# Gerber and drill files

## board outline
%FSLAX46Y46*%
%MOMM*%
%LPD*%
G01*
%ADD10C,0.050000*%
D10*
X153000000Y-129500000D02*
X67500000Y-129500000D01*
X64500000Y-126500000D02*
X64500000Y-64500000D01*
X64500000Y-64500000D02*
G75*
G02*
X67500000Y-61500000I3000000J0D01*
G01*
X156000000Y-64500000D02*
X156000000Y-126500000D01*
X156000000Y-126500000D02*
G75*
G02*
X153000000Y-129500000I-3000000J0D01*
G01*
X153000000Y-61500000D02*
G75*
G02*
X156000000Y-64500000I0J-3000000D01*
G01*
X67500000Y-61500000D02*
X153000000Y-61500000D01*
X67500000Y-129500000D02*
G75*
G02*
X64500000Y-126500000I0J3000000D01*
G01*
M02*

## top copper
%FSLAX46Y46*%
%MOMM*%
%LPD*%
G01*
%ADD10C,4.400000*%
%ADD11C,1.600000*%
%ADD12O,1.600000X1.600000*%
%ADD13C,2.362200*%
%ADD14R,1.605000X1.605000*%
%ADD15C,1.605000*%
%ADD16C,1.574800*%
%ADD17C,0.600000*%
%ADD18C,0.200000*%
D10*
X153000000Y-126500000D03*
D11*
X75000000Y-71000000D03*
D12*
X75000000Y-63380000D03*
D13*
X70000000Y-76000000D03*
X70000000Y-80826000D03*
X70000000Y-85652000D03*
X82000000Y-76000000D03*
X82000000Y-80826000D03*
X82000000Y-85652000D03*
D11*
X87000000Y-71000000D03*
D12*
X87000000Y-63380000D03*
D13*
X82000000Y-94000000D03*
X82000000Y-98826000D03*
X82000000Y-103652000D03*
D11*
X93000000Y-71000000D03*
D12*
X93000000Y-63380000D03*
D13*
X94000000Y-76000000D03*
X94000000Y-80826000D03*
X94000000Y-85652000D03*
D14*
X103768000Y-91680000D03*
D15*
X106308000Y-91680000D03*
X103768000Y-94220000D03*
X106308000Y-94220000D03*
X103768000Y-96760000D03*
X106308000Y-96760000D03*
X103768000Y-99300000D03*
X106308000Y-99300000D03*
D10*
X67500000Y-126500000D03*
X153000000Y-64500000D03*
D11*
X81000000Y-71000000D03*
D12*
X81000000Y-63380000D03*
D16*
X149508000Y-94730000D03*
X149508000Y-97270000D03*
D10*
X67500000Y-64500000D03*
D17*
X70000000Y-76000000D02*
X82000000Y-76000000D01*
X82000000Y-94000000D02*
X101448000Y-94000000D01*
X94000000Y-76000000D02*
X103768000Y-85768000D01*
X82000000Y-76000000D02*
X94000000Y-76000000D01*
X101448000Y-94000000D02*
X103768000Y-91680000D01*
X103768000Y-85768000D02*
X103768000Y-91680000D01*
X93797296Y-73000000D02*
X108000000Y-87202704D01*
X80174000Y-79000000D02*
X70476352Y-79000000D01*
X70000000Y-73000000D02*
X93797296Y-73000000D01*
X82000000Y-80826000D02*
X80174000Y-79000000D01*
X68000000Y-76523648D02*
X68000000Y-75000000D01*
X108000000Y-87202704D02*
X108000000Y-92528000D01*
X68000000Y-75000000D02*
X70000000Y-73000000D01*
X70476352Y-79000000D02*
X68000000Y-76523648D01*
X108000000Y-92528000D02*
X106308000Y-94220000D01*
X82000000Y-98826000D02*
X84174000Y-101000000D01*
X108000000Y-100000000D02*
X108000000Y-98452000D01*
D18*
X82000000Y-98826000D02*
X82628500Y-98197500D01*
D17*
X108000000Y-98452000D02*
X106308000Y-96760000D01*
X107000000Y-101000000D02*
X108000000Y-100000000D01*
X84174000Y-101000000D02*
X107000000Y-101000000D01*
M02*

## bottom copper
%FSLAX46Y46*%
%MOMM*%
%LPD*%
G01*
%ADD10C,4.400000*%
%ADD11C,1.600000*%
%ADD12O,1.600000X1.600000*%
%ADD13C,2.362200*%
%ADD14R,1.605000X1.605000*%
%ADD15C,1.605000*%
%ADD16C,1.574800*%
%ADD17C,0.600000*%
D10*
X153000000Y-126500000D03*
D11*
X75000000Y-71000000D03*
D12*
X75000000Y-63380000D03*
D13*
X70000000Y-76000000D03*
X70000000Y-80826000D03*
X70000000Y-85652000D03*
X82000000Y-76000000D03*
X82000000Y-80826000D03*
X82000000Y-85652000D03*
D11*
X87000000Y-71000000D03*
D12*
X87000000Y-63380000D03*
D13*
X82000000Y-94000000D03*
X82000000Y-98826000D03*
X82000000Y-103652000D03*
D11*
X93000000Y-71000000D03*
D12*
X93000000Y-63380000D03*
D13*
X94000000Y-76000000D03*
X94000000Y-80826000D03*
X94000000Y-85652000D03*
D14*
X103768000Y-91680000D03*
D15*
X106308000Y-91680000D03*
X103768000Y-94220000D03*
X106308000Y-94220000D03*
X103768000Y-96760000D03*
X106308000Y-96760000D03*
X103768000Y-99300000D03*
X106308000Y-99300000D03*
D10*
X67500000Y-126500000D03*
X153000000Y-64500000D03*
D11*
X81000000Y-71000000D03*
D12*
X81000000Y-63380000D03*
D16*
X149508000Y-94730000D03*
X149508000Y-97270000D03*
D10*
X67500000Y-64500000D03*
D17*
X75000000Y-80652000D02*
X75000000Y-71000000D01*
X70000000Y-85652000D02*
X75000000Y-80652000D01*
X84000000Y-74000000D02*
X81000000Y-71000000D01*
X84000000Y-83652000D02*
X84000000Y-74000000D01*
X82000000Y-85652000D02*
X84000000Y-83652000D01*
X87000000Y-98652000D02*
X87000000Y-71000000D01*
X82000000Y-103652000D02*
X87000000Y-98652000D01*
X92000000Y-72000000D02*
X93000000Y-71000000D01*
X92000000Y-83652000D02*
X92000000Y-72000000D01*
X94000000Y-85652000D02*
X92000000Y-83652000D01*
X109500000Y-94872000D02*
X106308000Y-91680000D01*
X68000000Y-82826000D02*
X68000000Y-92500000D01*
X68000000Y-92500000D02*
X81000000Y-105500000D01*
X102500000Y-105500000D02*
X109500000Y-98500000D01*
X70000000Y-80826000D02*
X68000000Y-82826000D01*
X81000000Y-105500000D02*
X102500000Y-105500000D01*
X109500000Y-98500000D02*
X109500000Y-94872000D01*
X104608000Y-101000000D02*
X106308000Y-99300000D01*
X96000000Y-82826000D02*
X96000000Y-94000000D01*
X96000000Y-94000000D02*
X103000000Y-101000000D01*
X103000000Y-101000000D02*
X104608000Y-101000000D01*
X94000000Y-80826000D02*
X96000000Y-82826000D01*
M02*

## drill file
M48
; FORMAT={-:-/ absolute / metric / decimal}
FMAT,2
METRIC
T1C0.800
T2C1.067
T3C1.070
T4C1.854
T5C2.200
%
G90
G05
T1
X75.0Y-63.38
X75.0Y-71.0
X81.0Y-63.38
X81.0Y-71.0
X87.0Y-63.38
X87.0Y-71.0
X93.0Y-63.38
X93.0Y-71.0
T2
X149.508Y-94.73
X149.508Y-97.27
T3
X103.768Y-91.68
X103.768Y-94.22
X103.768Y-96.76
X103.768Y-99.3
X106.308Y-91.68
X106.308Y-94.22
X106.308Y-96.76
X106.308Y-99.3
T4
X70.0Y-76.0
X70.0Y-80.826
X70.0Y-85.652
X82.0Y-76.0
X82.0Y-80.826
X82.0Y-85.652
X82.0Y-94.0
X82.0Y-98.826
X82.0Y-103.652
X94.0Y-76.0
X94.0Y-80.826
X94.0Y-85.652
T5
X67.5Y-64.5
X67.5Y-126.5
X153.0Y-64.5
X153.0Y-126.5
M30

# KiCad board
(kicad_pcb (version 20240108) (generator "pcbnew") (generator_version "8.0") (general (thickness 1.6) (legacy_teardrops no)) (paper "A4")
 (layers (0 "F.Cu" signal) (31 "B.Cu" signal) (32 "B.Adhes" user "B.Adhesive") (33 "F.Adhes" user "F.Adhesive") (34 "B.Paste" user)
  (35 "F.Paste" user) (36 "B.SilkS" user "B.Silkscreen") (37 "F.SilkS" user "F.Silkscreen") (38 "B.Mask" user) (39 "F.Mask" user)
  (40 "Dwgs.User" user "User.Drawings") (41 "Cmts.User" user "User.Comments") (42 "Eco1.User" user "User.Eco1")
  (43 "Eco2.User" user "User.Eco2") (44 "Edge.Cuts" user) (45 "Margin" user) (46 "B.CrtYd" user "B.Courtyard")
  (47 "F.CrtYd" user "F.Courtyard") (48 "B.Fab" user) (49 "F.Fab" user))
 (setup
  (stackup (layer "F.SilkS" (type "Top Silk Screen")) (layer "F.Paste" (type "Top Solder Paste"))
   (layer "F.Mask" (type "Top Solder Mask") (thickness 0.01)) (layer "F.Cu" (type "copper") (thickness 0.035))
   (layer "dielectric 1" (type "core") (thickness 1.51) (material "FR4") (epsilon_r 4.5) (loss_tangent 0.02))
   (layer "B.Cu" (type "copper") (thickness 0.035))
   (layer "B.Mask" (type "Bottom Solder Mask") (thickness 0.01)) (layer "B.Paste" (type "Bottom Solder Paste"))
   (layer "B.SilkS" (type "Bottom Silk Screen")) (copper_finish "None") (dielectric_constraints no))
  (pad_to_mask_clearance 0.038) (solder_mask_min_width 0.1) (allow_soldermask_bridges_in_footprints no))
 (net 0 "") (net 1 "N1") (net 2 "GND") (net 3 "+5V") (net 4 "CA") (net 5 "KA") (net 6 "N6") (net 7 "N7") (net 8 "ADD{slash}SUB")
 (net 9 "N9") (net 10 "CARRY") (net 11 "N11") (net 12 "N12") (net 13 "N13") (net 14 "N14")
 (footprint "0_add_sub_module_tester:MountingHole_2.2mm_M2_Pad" (layer "F.Cu") (at 153 126.5)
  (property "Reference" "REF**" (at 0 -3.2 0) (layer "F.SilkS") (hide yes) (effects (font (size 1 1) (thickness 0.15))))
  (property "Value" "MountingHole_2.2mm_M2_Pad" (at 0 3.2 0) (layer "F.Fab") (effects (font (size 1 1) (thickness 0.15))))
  (pad "1" thru_hole circle (at 0 0) (size 4.4 4.4) (drill 2.2) (layers "*.Cu" "*.Mask") (remove_unused_layers no)))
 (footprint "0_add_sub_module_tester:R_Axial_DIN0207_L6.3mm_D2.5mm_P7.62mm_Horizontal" (layer "F.Cu") (at 75 71 90)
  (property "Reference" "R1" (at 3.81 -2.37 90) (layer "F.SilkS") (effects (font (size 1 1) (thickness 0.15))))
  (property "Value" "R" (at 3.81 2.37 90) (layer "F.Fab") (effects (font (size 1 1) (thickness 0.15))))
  (pad "1" thru_hole circle (at 0 0 90) (size 1.6 1.6) (drill 0.8) (layers "*.Cu" "*.Mask") (remove_unused_layers no) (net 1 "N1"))
  (pad "2" thru_hole oval (at 7.62 0 90) (size 1.6 1.6) (drill 0.8) (layers "*.Cu" "*.Mask") (remove_unused_layers no) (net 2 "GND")))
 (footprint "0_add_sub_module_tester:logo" (layer "F.Cu") (at 127 95.5)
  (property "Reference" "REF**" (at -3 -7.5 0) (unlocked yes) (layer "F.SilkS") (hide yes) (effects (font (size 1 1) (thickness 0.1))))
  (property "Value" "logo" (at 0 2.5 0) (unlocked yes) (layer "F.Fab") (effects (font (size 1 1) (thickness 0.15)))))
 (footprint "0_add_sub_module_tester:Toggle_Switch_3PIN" (layer "F.Cu") (at 70 76 -90)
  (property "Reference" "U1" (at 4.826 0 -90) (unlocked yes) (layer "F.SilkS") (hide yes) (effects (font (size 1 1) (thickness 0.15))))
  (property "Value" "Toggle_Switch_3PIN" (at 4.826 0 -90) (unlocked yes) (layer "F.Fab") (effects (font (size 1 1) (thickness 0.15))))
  (pad "1" thru_hole circle (at 0 0 270) (size 2.3622 2.3622) (drill 1.8542) (layers "*.Cu" "*.Mask") (remove_unused_layers no)
   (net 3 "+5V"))
  (pad "2" thru_hole circle (at 4.826 0 270) (size 2.3622 2.3622) (drill 1.8542) (layers "*.Cu" "*.Mask") (remove_unused_layers no)
   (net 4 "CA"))
  (pad "3" thru_hole circle (at 9.652 0 270) (size 2.3622 2.3622) (drill 1.8542) (layers "*.Cu" "*.Mask") (remove_unused_layers no)
   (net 1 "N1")))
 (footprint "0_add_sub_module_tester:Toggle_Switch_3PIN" (layer "F.Cu") (at 82 76 -90)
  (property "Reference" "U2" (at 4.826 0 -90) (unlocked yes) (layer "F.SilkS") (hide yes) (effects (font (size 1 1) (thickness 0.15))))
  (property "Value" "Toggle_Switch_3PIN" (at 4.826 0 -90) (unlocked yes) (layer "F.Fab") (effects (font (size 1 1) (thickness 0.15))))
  (pad "1" thru_hole circle (at 0 0 270) (size 2.3622 2.3622) (drill 1.8542) (layers "*.Cu" "*.Mask") (remove_unused_layers no)
   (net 3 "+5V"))
  (pad "2" thru_hole circle (at 4.826 0 270) (size 2.3622 2.3622) (drill 1.8542) (layers "*.Cu" "*.Mask") (remove_unused_layers no)
   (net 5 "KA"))
  (pad "3" thru_hole circle (at 9.652 0 270) (size 2.3622 2.3622) (drill 1.8542) (layers "*.Cu" "*.Mask") (remove_unused_layers no)
   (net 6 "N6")))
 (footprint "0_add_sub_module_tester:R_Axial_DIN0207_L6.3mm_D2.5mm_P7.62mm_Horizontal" (layer "F.Cu") (at 87 71 90)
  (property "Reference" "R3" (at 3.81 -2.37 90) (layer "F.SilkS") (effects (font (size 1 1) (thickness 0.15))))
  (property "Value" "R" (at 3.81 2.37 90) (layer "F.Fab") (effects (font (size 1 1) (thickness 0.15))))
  (pad "1" thru_hole circle (at 0 0 90) (size 1.6 1.6) (drill 0.8) (layers "*.Cu" "*.Mask") (remove_unused_layers no) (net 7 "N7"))
  (pad "2" thru_hole oval (at 7.62 0 90) (size 1.6 1.6) (drill 0.8) (layers "*.Cu" "*.Mask") (remove_unused_layers no) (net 2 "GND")))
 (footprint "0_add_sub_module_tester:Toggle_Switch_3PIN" (layer "F.Cu") (at 82 94 -90)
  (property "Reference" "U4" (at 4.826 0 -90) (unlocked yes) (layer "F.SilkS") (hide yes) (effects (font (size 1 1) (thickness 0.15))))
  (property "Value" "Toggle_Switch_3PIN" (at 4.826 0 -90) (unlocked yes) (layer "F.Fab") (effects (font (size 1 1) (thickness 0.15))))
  (pad "1" thru_hole circle (at 0 0 270) (size 2.3622 2.3622) (drill 1.8542) (layers "*.Cu" "*.Mask") (remove_unused_layers no)
   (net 3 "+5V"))
  (pad "2" thru_hole circle (at 4.826 0 270) (size 2.3622 2.3622) (drill 1.8542) (layers "*.Cu" "*.Mask") (remove_unused_layers no)
   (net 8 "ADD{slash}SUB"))
  (pad "3" thru_hole circle (at 9.652 0 270) (size 2.3622 2.3622) (drill 1.8542) (layers "*.Cu" "*.Mask") (remove_unused_layers no)
   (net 7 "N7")))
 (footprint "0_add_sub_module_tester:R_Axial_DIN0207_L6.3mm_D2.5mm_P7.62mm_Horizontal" (layer "F.Cu") (at 93 71 90)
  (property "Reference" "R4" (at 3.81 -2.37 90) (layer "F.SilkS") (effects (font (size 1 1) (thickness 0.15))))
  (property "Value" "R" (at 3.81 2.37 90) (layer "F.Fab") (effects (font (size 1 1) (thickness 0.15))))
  (pad "1" thru_hole circle (at 0 0 90) (size 1.6 1.6) (drill 0.8) (layers "*.Cu" "*.Mask") (remove_unused_layers no) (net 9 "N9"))
  (pad "2" thru_hole oval (at 7.62 0 90) (size 1.6 1.6) (drill 0.8) (layers "*.Cu" "*.Mask") (remove_unused_layers no) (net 2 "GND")))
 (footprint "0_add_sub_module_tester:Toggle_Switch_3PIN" (layer "F.Cu") (at 94 76 -90)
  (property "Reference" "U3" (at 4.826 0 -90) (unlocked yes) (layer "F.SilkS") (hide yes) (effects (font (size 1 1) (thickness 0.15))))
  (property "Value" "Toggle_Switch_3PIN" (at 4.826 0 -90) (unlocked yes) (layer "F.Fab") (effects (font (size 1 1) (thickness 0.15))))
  (pad "1" thru_hole circle (at 0 0 270) (size 2.3622 2.3622) (drill 1.8542) (layers "*.Cu" "*.Mask") (remove_unused_layers no)
   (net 3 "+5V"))
  (pad "2" thru_hole circle (at 4.826 0 270) (size 2.3622 2.3622) (drill 1.8542) (layers "*.Cu" "*.Mask") (remove_unused_layers no)
   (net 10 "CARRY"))
  (pad "3" thru_hole circle (at 9.652 0 270) (size 2.3622 2.3622) (drill 1.8542) (layers "*.Cu" "*.Mask") (remove_unused_layers no)
   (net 9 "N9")))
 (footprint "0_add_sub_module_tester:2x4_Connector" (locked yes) (layer "F.Cu") (at 103.738 91.69 -90)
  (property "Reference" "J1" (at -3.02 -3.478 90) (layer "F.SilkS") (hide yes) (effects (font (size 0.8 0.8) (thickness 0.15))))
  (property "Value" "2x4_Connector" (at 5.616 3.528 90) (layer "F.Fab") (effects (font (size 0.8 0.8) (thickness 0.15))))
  (pad "1" thru_hole rect (at -0.01 -0.03 270) (size 1.605 1.605) (drill 1.07) (layers "*.Cu" "*.Mask") (remove_unused_layers no)
   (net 3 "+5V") (solder_mask_margin 0.102))
  (pad "2" thru_hole circle (at -0.01 -2.57 270) (size 1.605 1.605) (drill 1.07) (layers "*.Cu" "*.Mask") (remove_unused_layers no)
   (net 4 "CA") (solder_mask_margin 0.102))
  (pad "3" thru_hole circle (at 2.53 -0.03 270) (size 1.605 1.605) (drill 1.07) (layers "*.Cu" "*.Mask") (remove_unused_layers no)
   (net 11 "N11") (solder_mask_margin 0.102))
  (pad "4" thru_hole circle (at 2.53 -2.57 270) (size 1.605 1.605) (drill 1.07) (layers "*.Cu" "*.Mask") (remove_unused_layers no)
   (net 5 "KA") (solder_mask_margin 0.102))
  (pad "5" thru_hole circle (at 5.07 -0.03 270) (size 1.605 1.605) (drill 1.07) (layers "*.Cu" "*.Mask") (remove_unused_layers no)
   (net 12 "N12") (solder_mask_margin 0.102))
  (pad "6" thru_hole circle (at 5.07 -2.57 270) (size 1.605 1.605) (drill 1.07) (layers "*.Cu" "*.Mask") (remove_unused_layers no)
   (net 8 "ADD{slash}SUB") (solder_mask_margin 0.102))
  (pad "7" thru_hole circle (at 7.61 -0.03 270) (size 1.605 1.605) (drill 1.07) (layers "*.Cu" "*.Mask") (remove_unused_layers no)
   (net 2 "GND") (solder_mask_margin 0.102))
  (pad "8" thru_hole circle (at 7.61 -2.57 270) (size 1.605 1.605) (drill 1.07) (layers "*.Cu" "*.Mask") (remove_unused_layers no)
   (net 10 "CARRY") (solder_mask_margin 0.102)))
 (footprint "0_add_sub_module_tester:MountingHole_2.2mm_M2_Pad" (layer "F.Cu") (at 67.5 126.5)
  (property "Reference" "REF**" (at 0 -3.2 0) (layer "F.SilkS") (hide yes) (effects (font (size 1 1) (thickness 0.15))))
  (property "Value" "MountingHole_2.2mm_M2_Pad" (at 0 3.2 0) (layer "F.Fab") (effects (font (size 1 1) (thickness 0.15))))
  (pad "1" thru_hole circle (at 0 0) (size 4.4 4.4) (drill 2.2) (layers "*.Cu" "*.Mask") (remove_unused_layers no)))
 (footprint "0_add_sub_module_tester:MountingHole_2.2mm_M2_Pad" (layer "F.Cu") (at 153 64.5)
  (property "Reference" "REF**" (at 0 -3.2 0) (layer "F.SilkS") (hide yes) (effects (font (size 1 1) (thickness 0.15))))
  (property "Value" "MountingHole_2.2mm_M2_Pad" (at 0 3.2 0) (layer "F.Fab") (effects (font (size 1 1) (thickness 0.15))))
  (pad "1" thru_hole circle (at 0 0) (size 4.4 4.4) (drill 2.2) (layers "*.Cu" "*.Mask") (remove_unused_layers no)))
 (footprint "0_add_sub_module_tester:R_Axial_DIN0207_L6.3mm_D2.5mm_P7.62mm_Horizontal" (layer "F.Cu") (at 81 71 90)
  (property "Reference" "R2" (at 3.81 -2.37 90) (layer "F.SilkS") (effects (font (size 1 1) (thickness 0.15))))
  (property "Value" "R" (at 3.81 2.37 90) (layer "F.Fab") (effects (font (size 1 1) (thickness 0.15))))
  (pad "1" thru_hole circle (at 0 0 90) (size 1.6 1.6) (drill 0.8) (layers "*.Cu" "*.Mask") (remove_unused_layers no) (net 6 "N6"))
  (pad "2" thru_hole oval (at 7.62 0 90) (size 1.6 1.6) (drill 0.8) (layers "*.Cu" "*.Mask") (remove_unused_layers no) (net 2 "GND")))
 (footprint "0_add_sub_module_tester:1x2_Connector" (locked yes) (layer "F.Cu") (at 149.508 94.73 -90)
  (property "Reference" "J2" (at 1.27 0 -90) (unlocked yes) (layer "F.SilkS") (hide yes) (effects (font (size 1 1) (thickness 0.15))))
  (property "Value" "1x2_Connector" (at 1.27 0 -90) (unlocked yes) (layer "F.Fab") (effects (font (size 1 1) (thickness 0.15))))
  (pad "1" thru_hole circle (at 0 0 270) (size 1.5748 1.5748) (drill 1.0668) (layers "*.Cu" "*.Mask") (remove_unused_layers no)
   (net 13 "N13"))
  (pad "2" thru_hole circle (at 2.54 0 270) (size 1.5748 1.5748) (drill 1.0668) (layers "*.Cu" "*.Mask") (remove_unused_layers no)
   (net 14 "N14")))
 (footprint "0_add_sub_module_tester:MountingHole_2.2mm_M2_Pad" (layer "F.Cu") (at 67.5 64.5)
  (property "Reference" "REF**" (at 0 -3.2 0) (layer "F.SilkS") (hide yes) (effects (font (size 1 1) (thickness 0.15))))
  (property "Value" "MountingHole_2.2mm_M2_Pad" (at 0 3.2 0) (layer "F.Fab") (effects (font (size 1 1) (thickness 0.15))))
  (pad "1" thru_hole circle (at 0 0) (size 4.4 4.4) (drill 2.2) (layers "*.Cu" "*.Mask") (remove_unused_layers no)))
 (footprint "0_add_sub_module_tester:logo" (layer "B.Cu") (at 129.5 95.5 180)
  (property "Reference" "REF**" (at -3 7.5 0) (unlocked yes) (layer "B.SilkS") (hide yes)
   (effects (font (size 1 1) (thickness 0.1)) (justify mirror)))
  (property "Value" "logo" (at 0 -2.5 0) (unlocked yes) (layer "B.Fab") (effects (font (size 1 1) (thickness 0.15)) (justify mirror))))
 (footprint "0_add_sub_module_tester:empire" (layer "B.Cu") (at 141 112 180)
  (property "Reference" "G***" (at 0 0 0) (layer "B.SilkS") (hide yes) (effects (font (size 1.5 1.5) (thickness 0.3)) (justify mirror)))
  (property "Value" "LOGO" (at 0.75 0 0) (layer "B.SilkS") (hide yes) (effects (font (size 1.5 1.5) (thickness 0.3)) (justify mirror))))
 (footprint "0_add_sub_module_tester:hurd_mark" (layer "B.Cu") (at 106 68.75 180)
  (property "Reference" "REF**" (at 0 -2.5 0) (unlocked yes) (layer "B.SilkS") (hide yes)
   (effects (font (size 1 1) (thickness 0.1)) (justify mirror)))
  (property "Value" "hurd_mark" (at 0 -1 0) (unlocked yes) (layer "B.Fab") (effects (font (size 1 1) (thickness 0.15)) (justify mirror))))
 (gr_line (start 153 129.5) (end 67.5 129.5) (stroke (width 0.05) (type default)) (layer "Edge.Cuts"))
 (gr_line (start 64.5 126.5) (end 64.5 64.5) (stroke (width 0.05) (type default)) (layer "Edge.Cuts"))
 (gr_arc (start 64.5 64.5) (mid 65.37868 62.37868) (end 67.5 61.5) (stroke (width 0.05) (type default)) (layer "Edge.Cuts"))
 (gr_line (start 156 64.5) (end 156 126.5) (stroke (width 0.05) (type default)) (layer "Edge.Cuts"))
 (gr_arc (start 156 126.5) (mid 155.12132 128.62132) (end 153 129.5) (stroke (width 0.05) (type default)) (layer "Edge.Cuts"))
 (gr_arc (start 153 61.5) (mid 155.12132 62.37868) (end 156 64.5) (stroke (width 0.05) (type default)) (layer "Edge.Cuts"))
 (gr_line (start 67.5 61.5) (end 153 61.5) (stroke (width 0.05) (type default)) (layer "Edge.Cuts"))
 (gr_arc (start 67.5 129.5) (mid 65.37868 128.62132) (end 64.5 126.5) (stroke (width 0.05) (type default)) (layer "Edge.Cuts"))
 (segment (start 75 80.652) (end 75 71) (width 0.6) (layer "B.Cu") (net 1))
 (segment (start 70 85.652) (end 75 80.652) (width 0.6) (layer "B.Cu") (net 1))
 (segment (start 84 74) (end 81 71) (width 0.6) (layer "B.Cu") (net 6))
 (segment (start 84 83.652) (end 84 74) (width 0.6) (layer "B.Cu") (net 6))
 (segment (start 82 85.652) (end 84 83.652) (width 0.6) (layer "B.Cu") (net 6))
 (segment (start 87 98.652) (end 87 71) (width 0.6) (layer "B.Cu") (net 7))
 (segment (start 82 103.652) (end 87 98.652) (width 0.6) (layer "B.Cu") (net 7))
 (segment (start 92 72) (end 93 71) (width 0.6) (layer "B.Cu") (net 9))
 (segment (start 92 83.652) (end 92 72) (width 0.6) (layer "B.Cu") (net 9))
 (segment (start 94 85.652) (end 92 83.652) (width 0.6) (layer "B.Cu") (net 9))
 (segment (start 70 76) (end 82 76) (width 0.6) (layer "F.Cu") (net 3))
 (segment (start 82 94) (end 101.448 94) (width 0.6) (layer "F.Cu") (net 3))
 (segment (start 94 76) (end 103.768 85.768) (width 0.6) (layer "F.Cu") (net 3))
 (segment (start 82 76) (end 94 76) (width 0.6) (layer "F.Cu") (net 3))
 (segment (start 101.448 94) (end 103.768 91.68) (width 0.6) (layer "F.Cu") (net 3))
 (segment (start 103.768 85.768) (end 103.768 91.68) (width 0.6) (layer "F.Cu") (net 3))
 (segment (start 109.5 94.872) (end 106.308 91.68) (width 0.6) (layer "B.Cu") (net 4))
 (segment (start 68 82.826) (end 68 92.5) (width 0.6) (layer "B.Cu") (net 4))
 (segment (start 68 92.5) (end 81 105.5) (width 0.6) (layer "B.Cu") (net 4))
 (segment (start 102.5 105.5) (end 109.5 98.5) (width 0.6) (layer "B.Cu") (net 4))
 (segment (start 70 80.826) (end 68 82.826) (width 0.6) (layer "B.Cu") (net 4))
 (segment (start 81 105.5) (end 102.5 105.5) (width 0.6) (layer "B.Cu") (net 4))
 (segment (start 109.5 98.5) (end 109.5 94.872) (width 0.6) (layer "B.Cu") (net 4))
 (segment (start 93.797296 73) (end 108 87.202704) (width 0.6) (layer "F.Cu") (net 5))
 (segment (start 80.174 79) (end 70.476352 79) (width 0.6) (layer "F.Cu") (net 5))
 (segment (start 70 73) (end 93.797296 73) (width 0.6) (layer "F.Cu") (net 5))
 (segment (start 82 80.826) (end 80.174 79) (width 0.6) (layer "F.Cu") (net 5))
 (segment (start 68 76.523648) (end 68 75) (width 0.6) (layer "F.Cu") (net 5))
 (segment (start 108 87.202704) (end 108 92.528) (width 0.6) (layer "F.Cu") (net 5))
 (segment (start 68 75) (end 70 73) (width 0.6) (layer "F.Cu") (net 5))
 (segment (start 70.476352 79) (end 68 76.523648) (width 0.6) (layer "F.Cu") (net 5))
 (segment (start 108 92.528) (end 106.308 94.22) (width 0.6) (layer "F.Cu") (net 5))
 (segment (start 104.608 101) (end 106.308 99.3) (width 0.6) (layer "B.Cu") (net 10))
 (segment (start 96 82.826) (end 96 94) (width 0.6) (layer "B.Cu") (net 10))
 (segment (start 96 94) (end 103 101) (width 0.6) (layer "B.Cu") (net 10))
 (segment (start 103 101) (end 104.608 101) (width 0.6) (layer "B.Cu") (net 10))
 (segment (start 94 80.826) (end 96 82.826) (width 0.6) (layer "B.Cu") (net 10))
 (segment (start 82 98.826) (end 84.174 101) (width 0.6) (layer "F.Cu") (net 8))
 (segment (start 108 100) (end 108 98.452) (width 0.6) (layer "F.Cu") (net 8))
 (segment (start 82 98.826) (end 82.6285 98.1975) (width 0.2) (layer "F.Cu") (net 8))
 (segment (start 108 98.452) (end 106.308 96.76) (width 0.6) (layer "F.Cu") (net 8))
 (segment (start 107 101) (end 108 100) (width 0.6) (layer "F.Cu") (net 8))
 (segment (start 84.174 101) (end 107 101) (width 0.6) (layer "F.Cu") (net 8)))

